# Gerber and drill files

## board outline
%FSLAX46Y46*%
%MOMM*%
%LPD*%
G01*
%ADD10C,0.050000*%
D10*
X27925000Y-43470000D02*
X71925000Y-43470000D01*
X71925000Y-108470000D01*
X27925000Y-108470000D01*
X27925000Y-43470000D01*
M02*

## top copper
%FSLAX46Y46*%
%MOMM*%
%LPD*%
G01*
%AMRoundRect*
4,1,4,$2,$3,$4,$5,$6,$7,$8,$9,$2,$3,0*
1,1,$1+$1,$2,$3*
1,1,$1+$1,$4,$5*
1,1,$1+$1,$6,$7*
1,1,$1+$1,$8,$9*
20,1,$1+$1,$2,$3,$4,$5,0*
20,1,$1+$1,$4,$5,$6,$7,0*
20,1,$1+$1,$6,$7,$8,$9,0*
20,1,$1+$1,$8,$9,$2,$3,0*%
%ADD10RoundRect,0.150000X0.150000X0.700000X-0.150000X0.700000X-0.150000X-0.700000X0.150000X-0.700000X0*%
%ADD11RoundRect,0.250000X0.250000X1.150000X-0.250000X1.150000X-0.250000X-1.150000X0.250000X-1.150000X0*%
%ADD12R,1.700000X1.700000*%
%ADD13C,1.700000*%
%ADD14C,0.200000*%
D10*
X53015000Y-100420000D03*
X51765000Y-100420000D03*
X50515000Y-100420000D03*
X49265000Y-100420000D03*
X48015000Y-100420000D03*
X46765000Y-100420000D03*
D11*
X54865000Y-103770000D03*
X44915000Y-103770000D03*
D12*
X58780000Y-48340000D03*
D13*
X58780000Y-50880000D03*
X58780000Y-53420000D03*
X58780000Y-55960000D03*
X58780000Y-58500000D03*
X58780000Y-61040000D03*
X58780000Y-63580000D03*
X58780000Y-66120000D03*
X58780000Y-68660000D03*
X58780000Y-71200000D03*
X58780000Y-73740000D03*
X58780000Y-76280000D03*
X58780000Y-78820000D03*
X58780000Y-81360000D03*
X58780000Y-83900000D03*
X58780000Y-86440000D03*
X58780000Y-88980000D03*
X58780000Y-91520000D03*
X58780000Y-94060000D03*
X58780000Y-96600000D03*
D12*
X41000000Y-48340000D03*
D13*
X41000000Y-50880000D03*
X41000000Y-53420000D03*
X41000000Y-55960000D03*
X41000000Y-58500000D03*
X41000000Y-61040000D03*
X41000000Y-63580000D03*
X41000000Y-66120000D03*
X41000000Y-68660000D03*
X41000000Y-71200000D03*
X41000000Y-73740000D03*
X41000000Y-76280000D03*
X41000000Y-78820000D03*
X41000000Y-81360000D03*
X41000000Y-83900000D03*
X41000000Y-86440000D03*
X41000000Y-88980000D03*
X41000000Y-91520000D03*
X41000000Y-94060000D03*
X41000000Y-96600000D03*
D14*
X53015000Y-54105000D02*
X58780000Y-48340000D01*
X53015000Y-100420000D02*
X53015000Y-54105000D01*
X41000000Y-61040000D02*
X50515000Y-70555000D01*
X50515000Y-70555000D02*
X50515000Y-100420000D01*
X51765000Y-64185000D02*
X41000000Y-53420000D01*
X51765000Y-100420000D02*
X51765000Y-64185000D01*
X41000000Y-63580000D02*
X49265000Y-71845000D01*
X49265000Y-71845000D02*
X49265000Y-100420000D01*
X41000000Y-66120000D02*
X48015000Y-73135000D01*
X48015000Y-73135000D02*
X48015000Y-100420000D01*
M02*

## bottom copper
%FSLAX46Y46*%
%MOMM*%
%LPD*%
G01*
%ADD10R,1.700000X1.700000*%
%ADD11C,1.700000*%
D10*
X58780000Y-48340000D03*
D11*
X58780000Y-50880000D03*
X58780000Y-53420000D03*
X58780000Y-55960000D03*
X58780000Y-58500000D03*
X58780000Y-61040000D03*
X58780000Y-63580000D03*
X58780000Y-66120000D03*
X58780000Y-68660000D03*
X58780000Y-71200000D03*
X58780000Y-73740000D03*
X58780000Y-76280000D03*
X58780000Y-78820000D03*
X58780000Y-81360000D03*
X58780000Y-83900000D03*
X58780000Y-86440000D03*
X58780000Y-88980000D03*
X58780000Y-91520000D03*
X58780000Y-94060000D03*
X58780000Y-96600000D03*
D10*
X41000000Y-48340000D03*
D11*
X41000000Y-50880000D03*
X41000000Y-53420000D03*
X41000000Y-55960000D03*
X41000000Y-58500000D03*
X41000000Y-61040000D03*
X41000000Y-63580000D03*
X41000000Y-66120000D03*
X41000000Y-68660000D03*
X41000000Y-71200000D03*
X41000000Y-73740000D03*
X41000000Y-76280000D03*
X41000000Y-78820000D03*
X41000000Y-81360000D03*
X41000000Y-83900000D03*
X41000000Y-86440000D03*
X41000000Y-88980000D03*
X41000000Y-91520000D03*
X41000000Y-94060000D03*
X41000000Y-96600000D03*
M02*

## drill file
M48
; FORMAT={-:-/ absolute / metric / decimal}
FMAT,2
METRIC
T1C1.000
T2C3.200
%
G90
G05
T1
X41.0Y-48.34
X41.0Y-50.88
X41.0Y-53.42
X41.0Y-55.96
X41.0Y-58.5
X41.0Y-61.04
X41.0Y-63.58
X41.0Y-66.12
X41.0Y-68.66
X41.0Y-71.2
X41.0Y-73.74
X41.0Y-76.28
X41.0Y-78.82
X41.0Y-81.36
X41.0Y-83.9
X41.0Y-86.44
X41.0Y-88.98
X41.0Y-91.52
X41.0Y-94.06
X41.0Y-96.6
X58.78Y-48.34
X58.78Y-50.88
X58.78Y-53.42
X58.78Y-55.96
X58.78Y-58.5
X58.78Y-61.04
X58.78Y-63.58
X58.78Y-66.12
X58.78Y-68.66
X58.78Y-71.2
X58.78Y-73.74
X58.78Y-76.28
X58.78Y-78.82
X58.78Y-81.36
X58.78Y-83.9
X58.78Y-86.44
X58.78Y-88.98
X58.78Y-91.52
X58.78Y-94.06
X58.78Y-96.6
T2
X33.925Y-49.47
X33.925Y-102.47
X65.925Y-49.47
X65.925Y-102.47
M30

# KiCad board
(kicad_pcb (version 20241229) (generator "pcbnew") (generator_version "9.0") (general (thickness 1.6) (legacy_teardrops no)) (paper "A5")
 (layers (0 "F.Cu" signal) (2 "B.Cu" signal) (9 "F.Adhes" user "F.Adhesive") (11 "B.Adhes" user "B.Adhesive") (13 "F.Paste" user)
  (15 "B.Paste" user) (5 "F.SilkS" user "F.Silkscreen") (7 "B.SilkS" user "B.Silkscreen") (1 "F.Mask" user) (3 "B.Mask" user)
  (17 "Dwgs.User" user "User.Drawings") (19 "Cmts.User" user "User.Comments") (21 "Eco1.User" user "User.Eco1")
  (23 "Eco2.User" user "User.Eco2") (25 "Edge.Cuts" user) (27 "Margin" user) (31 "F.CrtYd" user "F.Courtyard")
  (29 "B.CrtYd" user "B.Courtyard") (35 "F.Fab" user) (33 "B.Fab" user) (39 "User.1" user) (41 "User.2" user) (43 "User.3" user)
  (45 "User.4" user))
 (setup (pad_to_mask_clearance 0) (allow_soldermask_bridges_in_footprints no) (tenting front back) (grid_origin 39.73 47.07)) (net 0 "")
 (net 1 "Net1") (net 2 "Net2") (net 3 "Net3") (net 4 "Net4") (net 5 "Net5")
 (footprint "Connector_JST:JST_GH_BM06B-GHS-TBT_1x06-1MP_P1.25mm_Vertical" (layer "F.Cu") (at 49.89 102.37 180)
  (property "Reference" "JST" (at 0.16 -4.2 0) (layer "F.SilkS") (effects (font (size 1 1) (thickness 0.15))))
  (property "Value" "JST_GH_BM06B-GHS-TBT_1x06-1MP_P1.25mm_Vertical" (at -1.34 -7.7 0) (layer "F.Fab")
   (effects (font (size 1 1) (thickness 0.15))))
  (pad "1" smd roundrect (at -3.125 1.95 180) (size 0.6 1.7) (layers "F.Cu" "F.Mask" "F.Paste") (roundrect_rratio 0.25) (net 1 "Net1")
   (solder_mask_margin 0))
  (pad "2" smd roundrect (at -1.875 1.95 180) (size 0.6 1.7) (layers "F.Cu" "F.Mask" "F.Paste") (roundrect_rratio 0.25) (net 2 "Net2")
   (solder_mask_margin 0))
  (pad "3" smd roundrect (at -0.625 1.95 180) (size 0.6 1.7) (layers "F.Cu" "F.Mask" "F.Paste") (roundrect_rratio 0.25) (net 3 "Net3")
   (solder_mask_margin 0))
  (pad "4" smd roundrect (at 0.625 1.95 180) (size 0.6 1.7) (layers "F.Cu" "F.Mask" "F.Paste") (roundrect_rratio 0.25) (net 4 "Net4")
   (solder_mask_margin 0))
  (pad "5" smd roundrect (at 1.875 1.95 180) (size 0.6 1.7) (layers "F.Cu" "F.Mask" "F.Paste") (roundrect_rratio 0.25) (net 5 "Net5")
   (solder_mask_margin 0))
  (pad "6" smd roundrect (at 3.125 1.95 180) (size 0.6 1.7) (layers "F.Cu" "F.Mask" "F.Paste") (roundrect_rratio 0.25))
  (pad "MP" smd roundrect (at -4.975 -1.4 180) (size 1 2.8) (layers "F.Cu" "F.Mask" "F.Paste") (roundrect_rratio 0.25))
  (pad "MP" smd roundrect (at 4.975 -1.4 180) (size 1 2.8) (layers "F.Cu" "F.Mask" "F.Paste") (roundrect_rratio 0.25)))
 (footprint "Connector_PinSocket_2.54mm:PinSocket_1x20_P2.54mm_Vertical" (layer "F.Cu") (at 58.78 48.34)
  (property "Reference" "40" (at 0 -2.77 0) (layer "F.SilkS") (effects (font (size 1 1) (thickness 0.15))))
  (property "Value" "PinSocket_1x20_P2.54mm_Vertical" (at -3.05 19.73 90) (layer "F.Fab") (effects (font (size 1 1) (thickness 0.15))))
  (pad "1" thru_hole rect (at 0 0) (size 1.7 1.7) (drill 1) (layers "*.Cu" "*.Mask") (remove_unused_layers no) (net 1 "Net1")
   (solder_mask_margin 0))
  (pad "2" thru_hole circle (at 0 2.54) (size 1.7 1.7) (drill 1) (layers "*.Cu" "*.Mask") (remove_unused_layers no))
  (pad "3" thru_hole circle (at 0 5.08) (size 1.7 1.7) (drill 1) (layers "*.Cu" "*.Mask") (remove_unused_layers no))
  (pad "4" thru_hole circle (at 0 7.62) (size 1.7 1.7) (drill 1) (layers "*.Cu" "*.Mask") (remove_unused_layers no))
  (pad "5" thru_hole circle (at 0 10.16) (size 1.7 1.7) (drill 1) (layers "*.Cu" "*.Mask") (remove_unused_layers no))
  (pad "6" thru_hole circle (at 0 12.7) (size 1.7 1.7) (drill 1) (layers "*.Cu" "*.Mask") (remove_unused_layers no))
  (pad "7" thru_hole circle (at 0 15.24) (size 1.7 1.7) (drill 1) (layers "*.Cu" "*.Mask") (remove_unused_layers no))
  (pad "8" thru_hole circle (at 0 17.78) (size 1.7 1.7) (drill 1) (layers "*.Cu" "*.Mask") (remove_unused_layers no))
  (pad "9" thru_hole circle (at 0 20.32) (size 1.7 1.7) (drill 1) (layers "*.Cu" "*.Mask") (remove_unused_layers no))
  (pad "10" thru_hole circle (at 0 22.86) (size 1.7 1.7) (drill 1) (layers "*.Cu" "*.Mask") (remove_unused_layers no))
  (pad "11" thru_hole circle (at 0 25.4) (size 1.7 1.7) (drill 1) (layers "*.Cu" "*.Mask") (remove_unused_layers no))
  (pad "12" thru_hole circle (at 0 27.94) (size 1.7 1.7) (drill 1) (layers "*.Cu" "*.Mask") (remove_unused_layers no))
  (pad "13" thru_hole circle (at 0 30.48) (size 1.7 1.7) (drill 1) (layers "*.Cu" "*.Mask") (remove_unused_layers no))
  (pad "14" thru_hole circle (at 0 33.02) (size 1.7 1.7) (drill 1) (layers "*.Cu" "*.Mask") (remove_unused_layers no))
  (pad "15" thru_hole circle (at 0 35.56) (size 1.7 1.7) (drill 1) (layers "*.Cu" "*.Mask") (remove_unused_layers no))
  (pad "16" thru_hole circle (at 0 38.1) (size 1.7 1.7) (drill 1) (layers "*.Cu" "*.Mask") (remove_unused_layers no))
  (pad "17" thru_hole circle (at 0 40.64) (size 1.7 1.7) (drill 1) (layers "*.Cu" "*.Mask") (remove_unused_layers no))
  (pad "18" thru_hole circle (at 0 43.18) (size 1.7 1.7) (drill 1) (layers "*.Cu" "*.Mask") (remove_unused_layers no))
  (pad "19" thru_hole circle (at 0 45.72) (size 1.7 1.7) (drill 1) (layers "*.Cu" "*.Mask") (remove_unused_layers no))
  (pad "20" thru_hole circle (at 0 48.26) (size 1.7 1.7) (drill 1) (layers "*.Cu" "*.Mask") (remove_unused_layers no)))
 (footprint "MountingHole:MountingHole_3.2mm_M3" (layer "F.Cu") (at 65.925 102.47)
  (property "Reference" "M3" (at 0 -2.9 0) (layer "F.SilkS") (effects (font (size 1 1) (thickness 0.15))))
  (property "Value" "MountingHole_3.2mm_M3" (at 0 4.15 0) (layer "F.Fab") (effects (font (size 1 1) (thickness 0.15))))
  (pad "" np_thru_hole circle (at 0 0) (size 3.2 3.2) (drill 3.2) (layers "*.Cu" "*.Mask")))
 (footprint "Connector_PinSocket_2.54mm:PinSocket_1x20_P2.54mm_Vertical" (layer "F.Cu") (at 41 48.34)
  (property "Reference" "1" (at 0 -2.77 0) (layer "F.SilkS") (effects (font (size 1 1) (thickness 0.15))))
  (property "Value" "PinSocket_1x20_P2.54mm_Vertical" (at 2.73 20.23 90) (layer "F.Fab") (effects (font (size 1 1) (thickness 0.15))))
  (pad "1" thru_hole rect (at 0 0) (size 1.7 1.7) (drill 1) (layers "*.Cu" "*.Mask") (remove_unused_layers no))
  (pad "2" thru_hole circle (at 0 2.54) (size 1.7 1.7) (drill 1) (layers "*.Cu" "*.Mask") (remove_unused_layers no))
  (pad "3" thru_hole circle (at 0 5.08) (size 1.7 1.7) (drill 1) (layers "*.Cu" "*.Mask") (remove_unused_layers no) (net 2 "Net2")
   (solder_mask_margin 0))
  (pad "4" thru_hole circle (at 0 7.62) (size 1.7 1.7) (drill 1) (layers "*.Cu" "*.Mask") (remove_unused_layers no))
  (pad "5" thru_hole circle (at 0 10.16) (size 1.7 1.7) (drill 1) (layers "*.Cu" "*.Mask") (remove_unused_layers no))
  (pad "6" thru_hole circle (at 0 12.7) (size 1.7 1.7) (drill 1) (layers "*.Cu" "*.Mask") (remove_unused_layers no) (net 3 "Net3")
   (solder_mask_margin 0))
  (pad "7" thru_hole circle (at 0 15.24) (size 1.7 1.7) (drill 1) (layers "*.Cu" "*.Mask") (remove_unused_layers no) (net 4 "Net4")
   (clearance 0))
  (pad "8" thru_hole circle (at 0 17.78) (size 1.7 1.7) (drill 1) (layers "*.Cu" "*.Mask") (remove_unused_layers no) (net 5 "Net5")
   (solder_mask_margin 0))
  (pad "9" thru_hole circle (at 0 20.32) (size 1.7 1.7) (drill 1) (layers "*.Cu" "*.Mask") (remove_unused_layers no))
  (pad "10" thru_hole circle (at 0 22.86) (size 1.7 1.7) (drill 1) (layers "*.Cu" "*.Mask") (remove_unused_layers no))
  (pad "11" thru_hole circle (at 0 25.4) (size 1.7 1.7) (drill 1) (layers "*.Cu" "*.Mask") (remove_unused_layers no))
  (pad "12" thru_hole circle (at 0 27.94) (size 1.7 1.7) (drill 1) (layers "*.Cu" "*.Mask") (remove_unused_layers no))
  (pad "13" thru_hole circle (at 0 30.48) (size 1.7 1.7) (drill 1) (layers "*.Cu" "*.Mask") (remove_unused_layers no))
  (pad "14" thru_hole circle (at 0 33.02) (size 1.7 1.7) (drill 1) (layers "*.Cu" "*.Mask") (remove_unused_layers no))
  (pad "15" thru_hole circle (at 0 35.56) (size 1.7 1.7) (drill 1) (layers "*.Cu" "*.Mask") (remove_unused_layers no))
  (pad "16" thru_hole circle (at 0 38.1) (size 1.7 1.7) (drill 1) (layers "*.Cu" "*.Mask") (remove_unused_layers no))
  (pad "17" thru_hole circle (at 0 40.64) (size 1.7 1.7) (drill 1) (layers "*.Cu" "*.Mask") (remove_unused_layers no))
  (pad "18" thru_hole circle (at 0 43.18) (size 1.7 1.7) (drill 1) (layers "*.Cu" "*.Mask") (remove_unused_layers no))
  (pad "19" thru_hole circle (at 0 45.72) (size 1.7 1.7) (drill 1) (layers "*.Cu" "*.Mask") (remove_unused_layers no))
  (pad "20" thru_hole circle (at 0 48.26) (size 1.7 1.7) (drill 1) (layers "*.Cu" "*.Mask") (remove_unused_layers no)))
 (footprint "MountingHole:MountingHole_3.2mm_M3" (layer "F.Cu") (at 33.925 102.47)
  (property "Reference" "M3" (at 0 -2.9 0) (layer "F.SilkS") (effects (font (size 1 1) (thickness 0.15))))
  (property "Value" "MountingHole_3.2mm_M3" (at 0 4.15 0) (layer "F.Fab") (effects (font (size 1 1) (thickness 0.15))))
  (pad "" np_thru_hole circle (at 0 0) (size 3.2 3.2) (drill 3.2) (layers "*.Cu" "*.Mask")))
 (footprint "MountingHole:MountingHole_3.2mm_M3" (layer "F.Cu") (at 65.925 49.47)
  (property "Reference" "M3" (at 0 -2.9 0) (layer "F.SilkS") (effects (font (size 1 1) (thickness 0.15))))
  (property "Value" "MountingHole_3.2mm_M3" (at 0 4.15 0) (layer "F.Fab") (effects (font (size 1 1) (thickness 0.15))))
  (pad "" np_thru_hole circle (at 0 0) (size 3.2 3.2) (drill 3.2) (layers "*.Cu" "*.Mask")))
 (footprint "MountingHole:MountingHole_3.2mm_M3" (layer "F.Cu") (at 33.925 49.47)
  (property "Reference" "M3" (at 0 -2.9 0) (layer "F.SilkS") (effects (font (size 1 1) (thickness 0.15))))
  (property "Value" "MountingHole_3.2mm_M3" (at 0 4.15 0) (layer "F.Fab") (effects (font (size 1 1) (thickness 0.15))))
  (pad "" np_thru_hole circle (at 0 0) (size 3.2 3.2) (drill 3.2) (layers "*.Cu" "*.Mask")))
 (gr_rect (start 27.925 43.47) (end 71.925 108.47) (stroke (width 0.05) (type solid)) (fill no) (layer "Edge.Cuts"))
 (segment (start 53.015 54.105) (end 58.78 48.34) (width 0.2) (layer "F.Cu") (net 1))
 (segment (start 53.015 100.42) (end 53.015 54.105) (width 0.2) (layer "F.Cu") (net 1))
 (segment (start 41 61.04) (end 50.515 70.555) (width 0.2) (layer "F.Cu") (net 3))
 (segment (start 50.515 70.555) (end 50.515 100.42) (width 0.2) (layer "F.Cu") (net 3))
 (segment (start 51.765 64.185) (end 41 53.42) (width 0.2) (layer "F.Cu") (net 2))
 (segment (start 51.765 100.42) (end 51.765 64.185) (width 0.2) (layer "F.Cu") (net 2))
 (segment (start 41 63.58) (end 49.265 71.845) (width 0.2) (layer "F.Cu") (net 4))
 (segment (start 49.265 71.845) (end 49.265 100.42) (width 0.2) (layer "F.Cu") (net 4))
 (segment (start 41 66.12) (end 48.015 73.135) (width 0.2) (layer "F.Cu") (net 5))
 (segment (start 48.015 73.135) (end 48.015 100.42) (width 0.2) (layer "F.Cu") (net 5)))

